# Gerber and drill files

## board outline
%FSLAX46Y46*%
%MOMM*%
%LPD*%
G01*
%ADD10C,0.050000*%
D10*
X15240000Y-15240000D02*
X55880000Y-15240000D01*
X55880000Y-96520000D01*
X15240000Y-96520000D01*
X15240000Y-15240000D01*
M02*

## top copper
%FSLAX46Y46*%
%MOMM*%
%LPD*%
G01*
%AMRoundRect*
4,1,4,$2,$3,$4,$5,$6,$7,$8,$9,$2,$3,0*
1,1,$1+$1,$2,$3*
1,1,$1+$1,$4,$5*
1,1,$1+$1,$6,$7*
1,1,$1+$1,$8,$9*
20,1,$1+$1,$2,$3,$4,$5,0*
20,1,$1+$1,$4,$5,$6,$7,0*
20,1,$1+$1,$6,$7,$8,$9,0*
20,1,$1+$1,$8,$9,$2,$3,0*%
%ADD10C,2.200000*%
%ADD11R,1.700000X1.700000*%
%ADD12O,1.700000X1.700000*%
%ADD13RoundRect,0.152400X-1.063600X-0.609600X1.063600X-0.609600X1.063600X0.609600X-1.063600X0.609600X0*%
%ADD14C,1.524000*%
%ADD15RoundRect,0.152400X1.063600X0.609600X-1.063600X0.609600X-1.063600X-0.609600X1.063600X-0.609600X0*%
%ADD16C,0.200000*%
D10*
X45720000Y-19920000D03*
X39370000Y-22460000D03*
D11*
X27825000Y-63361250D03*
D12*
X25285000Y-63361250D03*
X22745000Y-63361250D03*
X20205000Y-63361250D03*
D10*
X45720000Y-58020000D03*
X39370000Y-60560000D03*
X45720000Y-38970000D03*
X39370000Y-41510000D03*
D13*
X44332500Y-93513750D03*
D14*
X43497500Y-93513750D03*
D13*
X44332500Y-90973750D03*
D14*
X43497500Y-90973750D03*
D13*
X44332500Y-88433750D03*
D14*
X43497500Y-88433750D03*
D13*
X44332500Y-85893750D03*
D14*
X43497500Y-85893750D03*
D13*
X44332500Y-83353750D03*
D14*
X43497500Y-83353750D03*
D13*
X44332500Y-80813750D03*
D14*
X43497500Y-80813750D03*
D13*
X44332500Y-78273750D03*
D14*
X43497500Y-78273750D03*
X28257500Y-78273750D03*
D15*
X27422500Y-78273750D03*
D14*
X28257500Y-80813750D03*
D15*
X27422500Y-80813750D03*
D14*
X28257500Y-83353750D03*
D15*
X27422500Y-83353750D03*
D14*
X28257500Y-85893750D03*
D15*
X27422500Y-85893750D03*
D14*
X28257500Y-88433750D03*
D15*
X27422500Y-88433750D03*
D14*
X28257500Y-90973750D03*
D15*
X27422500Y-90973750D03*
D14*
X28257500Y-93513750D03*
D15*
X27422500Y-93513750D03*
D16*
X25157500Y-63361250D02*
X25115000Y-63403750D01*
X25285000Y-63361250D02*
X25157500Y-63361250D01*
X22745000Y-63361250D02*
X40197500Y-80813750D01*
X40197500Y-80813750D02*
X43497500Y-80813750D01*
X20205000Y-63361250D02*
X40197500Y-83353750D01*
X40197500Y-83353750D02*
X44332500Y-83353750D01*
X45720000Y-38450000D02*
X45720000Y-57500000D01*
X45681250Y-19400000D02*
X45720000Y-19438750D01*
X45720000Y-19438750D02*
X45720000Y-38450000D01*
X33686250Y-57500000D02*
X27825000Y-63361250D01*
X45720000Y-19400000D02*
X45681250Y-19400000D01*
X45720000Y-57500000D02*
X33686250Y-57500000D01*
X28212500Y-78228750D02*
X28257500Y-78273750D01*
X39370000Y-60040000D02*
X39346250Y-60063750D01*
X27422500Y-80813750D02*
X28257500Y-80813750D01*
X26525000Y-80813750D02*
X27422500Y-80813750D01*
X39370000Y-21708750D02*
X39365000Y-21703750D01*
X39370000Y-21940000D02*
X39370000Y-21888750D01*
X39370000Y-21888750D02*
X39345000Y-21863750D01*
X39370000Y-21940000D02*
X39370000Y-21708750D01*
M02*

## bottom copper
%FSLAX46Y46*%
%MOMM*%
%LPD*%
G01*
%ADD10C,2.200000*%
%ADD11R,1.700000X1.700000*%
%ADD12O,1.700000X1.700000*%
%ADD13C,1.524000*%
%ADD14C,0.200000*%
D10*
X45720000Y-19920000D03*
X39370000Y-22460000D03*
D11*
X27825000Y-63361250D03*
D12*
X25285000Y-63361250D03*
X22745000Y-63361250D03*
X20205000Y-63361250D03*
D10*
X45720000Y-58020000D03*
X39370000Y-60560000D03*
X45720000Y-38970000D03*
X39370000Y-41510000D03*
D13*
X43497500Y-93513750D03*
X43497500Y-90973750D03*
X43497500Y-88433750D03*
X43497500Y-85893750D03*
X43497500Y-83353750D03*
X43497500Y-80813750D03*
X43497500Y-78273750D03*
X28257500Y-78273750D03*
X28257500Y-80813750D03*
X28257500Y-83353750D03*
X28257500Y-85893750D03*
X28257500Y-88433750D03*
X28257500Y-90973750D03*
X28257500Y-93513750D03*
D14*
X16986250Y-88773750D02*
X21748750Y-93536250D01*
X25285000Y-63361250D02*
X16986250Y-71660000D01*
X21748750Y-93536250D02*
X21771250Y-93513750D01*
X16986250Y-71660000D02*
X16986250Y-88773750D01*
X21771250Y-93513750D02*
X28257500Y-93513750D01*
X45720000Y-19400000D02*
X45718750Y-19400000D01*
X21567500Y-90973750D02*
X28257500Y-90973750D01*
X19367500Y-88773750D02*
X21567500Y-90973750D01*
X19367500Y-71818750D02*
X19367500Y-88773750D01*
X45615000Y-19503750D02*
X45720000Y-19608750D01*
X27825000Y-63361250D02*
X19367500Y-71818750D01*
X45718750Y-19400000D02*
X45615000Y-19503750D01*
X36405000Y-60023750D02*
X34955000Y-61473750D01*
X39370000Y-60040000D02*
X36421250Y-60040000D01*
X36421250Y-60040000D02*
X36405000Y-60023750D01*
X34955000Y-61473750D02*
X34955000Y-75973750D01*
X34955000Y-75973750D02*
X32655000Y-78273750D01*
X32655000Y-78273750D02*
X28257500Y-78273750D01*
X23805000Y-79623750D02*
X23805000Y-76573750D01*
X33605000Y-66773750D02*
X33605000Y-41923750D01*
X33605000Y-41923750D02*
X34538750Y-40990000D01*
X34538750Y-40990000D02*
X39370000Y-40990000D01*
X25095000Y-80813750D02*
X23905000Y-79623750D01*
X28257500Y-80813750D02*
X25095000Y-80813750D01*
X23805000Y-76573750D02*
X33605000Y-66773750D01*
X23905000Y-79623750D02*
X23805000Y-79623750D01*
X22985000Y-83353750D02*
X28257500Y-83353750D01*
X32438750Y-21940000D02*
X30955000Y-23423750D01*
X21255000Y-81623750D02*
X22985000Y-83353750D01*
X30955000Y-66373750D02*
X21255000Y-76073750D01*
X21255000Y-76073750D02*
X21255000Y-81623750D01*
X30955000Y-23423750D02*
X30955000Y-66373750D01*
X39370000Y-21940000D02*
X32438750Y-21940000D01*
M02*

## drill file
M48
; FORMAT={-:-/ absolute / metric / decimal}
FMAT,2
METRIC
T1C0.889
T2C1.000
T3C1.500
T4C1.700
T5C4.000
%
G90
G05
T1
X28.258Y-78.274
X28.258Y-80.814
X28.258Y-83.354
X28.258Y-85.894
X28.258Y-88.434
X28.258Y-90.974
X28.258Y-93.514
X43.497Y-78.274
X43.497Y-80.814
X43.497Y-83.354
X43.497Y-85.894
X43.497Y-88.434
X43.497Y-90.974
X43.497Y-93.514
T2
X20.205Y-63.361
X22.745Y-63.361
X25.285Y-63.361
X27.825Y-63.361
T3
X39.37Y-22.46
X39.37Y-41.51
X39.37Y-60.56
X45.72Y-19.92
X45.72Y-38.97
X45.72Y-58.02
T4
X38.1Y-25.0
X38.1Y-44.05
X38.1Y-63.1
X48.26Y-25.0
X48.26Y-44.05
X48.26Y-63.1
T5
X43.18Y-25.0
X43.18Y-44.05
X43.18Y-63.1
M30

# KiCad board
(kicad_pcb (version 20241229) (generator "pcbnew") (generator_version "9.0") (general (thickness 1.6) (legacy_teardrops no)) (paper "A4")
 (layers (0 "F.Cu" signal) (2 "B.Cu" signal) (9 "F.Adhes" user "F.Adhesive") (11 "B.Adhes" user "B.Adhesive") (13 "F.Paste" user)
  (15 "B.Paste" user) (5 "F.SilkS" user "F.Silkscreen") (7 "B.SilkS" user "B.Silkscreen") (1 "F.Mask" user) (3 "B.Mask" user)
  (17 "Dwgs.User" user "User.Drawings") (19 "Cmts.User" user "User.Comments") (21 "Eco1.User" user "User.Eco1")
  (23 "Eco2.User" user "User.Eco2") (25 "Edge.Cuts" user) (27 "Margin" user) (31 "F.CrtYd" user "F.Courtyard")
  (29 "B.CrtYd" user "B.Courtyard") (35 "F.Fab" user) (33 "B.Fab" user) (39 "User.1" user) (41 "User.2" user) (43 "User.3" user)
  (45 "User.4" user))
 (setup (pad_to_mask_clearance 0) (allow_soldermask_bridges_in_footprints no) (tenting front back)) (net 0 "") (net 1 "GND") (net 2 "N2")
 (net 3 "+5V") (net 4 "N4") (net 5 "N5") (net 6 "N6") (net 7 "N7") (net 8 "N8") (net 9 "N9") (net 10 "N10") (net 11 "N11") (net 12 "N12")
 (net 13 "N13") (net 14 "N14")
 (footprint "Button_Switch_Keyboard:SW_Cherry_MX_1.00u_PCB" (layer "F.Cu") (at 45.72 19.92)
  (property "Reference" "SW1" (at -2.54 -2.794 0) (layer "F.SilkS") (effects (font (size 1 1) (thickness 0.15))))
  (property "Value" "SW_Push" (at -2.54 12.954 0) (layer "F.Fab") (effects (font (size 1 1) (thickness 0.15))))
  (pad "" np_thru_hole circle (at -7.62 5.08) (size 1.7 1.7) (drill 1.7) (layers "*.Cu" "*.Mask"))
  (pad "" np_thru_hole circle (at -2.54 5.08) (size 4 4) (drill 4) (layers "*.Cu" "*.Mask"))
  (pad "" np_thru_hole circle (at 2.54 5.08) (size 1.7 1.7) (drill 1.7) (layers "*.Cu" "*.Mask"))
  (pad "1" thru_hole circle (at 0 0) (size 2.2 2.2) (drill 1.5) (layers "*.Cu" "*.Mask") (remove_unused_layers no) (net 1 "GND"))
  (pad "2" thru_hole circle (at -6.35 2.54) (size 2.2 2.2) (drill 1.5) (layers "*.Cu" "*.Mask") (remove_unused_layers no) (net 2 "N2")))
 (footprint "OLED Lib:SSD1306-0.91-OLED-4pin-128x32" (layer "F.Cu") (at 30.015 26.86125 -90)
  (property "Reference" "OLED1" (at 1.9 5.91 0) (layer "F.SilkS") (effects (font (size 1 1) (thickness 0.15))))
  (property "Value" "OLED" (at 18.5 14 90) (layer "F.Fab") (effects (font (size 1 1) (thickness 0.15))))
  (pad "1" thru_hole rect (at 36.5 2.19 270) (size 1.7 1.7) (drill 1) (layers "*.Cu" "*.Mask") (remove_unused_layers no) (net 1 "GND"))
  (pad "2" thru_hole oval (at 36.5 4.73 270) (size 1.7 1.7) (drill 1) (layers "*.Cu" "*.Mask") (remove_unused_layers no) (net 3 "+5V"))
  (pad "3" thru_hole oval (at 36.5 7.27 270) (size 1.7 1.7) (drill 1) (layers "*.Cu" "*.Mask") (remove_unused_layers no) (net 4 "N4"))
  (pad "4" thru_hole oval (at 36.5 9.81 270) (size 1.7 1.7) (drill 1) (layers "*.Cu" "*.Mask") (remove_unused_layers no) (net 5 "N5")))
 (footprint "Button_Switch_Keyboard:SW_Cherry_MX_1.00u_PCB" (layer "F.Cu") (at 45.72 58.02)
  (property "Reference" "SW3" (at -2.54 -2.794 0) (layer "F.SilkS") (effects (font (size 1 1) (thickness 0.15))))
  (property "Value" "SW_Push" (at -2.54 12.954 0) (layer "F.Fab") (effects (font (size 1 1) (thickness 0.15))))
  (pad "" np_thru_hole circle (at -7.62 5.08) (size 1.7 1.7) (drill 1.7) (layers "*.Cu" "*.Mask"))
  (pad "" np_thru_hole circle (at -2.54 5.08) (size 4 4) (drill 4) (layers "*.Cu" "*.Mask"))
  (pad "" np_thru_hole circle (at 2.54 5.08) (size 1.7 1.7) (drill 1.7) (layers "*.Cu" "*.Mask"))
  (pad "1" thru_hole circle (at 0 0) (size 2.2 2.2) (drill 1.5) (layers "*.Cu" "*.Mask") (remove_unused_layers no) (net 1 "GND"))
  (pad "2" thru_hole circle (at -6.35 2.54) (size 2.2 2.2) (drill 1.5) (layers "*.Cu" "*.Mask") (remove_unused_layers no) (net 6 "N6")))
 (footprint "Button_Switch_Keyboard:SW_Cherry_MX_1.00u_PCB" (layer "F.Cu") (at 45.72 38.97)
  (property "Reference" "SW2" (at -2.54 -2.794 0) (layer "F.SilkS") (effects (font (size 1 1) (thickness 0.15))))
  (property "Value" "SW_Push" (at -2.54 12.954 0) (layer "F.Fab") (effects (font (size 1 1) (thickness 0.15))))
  (pad "" np_thru_hole circle (at -7.62 5.08) (size 1.7 1.7) (drill 1.7) (layers "*.Cu" "*.Mask"))
  (pad "" np_thru_hole circle (at -2.54 5.08) (size 4 4) (drill 4) (layers "*.Cu" "*.Mask"))
  (pad "" np_thru_hole circle (at 2.54 5.08) (size 1.7 1.7) (drill 1.7) (layers "*.Cu" "*.Mask"))
  (pad "1" thru_hole circle (at 0 0) (size 2.2 2.2) (drill 1.5) (layers "*.Cu" "*.Mask") (remove_unused_layers no) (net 1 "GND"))
  (pad "2" thru_hole circle (at -6.35 2.54) (size 2.2 2.2) (drill 1.5) (layers "*.Cu" "*.Mask") (remove_unused_layers no) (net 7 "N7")))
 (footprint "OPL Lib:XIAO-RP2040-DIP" (layer "F.Cu") (at 35.8775 85.89375 180)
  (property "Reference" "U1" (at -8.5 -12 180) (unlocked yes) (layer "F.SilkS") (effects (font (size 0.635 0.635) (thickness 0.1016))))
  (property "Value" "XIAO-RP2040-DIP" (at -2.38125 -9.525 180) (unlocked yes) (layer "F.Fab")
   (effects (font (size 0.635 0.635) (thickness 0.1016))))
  (pad "1" smd roundrect (at -8.455 -7.62) (size 2.432 1.524) (layers "F.Cu" "F.Mask") (roundrect_rratio 0.1) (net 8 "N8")
   (thermal_bridge_angle 45))
  (pad "1" thru_hole circle (at -7.62 -7.62) (size 1.524 1.524) (drill 0.889) (layers "*.Cu" "*.Mask") (remove_unused_layers no)
   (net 8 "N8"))
  (pad "2" smd roundrect (at -8.455 -5.08) (size 2.432 1.524) (layers "F.Cu" "F.Mask") (roundrect_rratio 0.1) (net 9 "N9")
   (thermal_bridge_angle 45))
  (pad "2" thru_hole circle (at -7.62 -5.08) (size 1.524 1.524) (drill 0.889) (layers "*.Cu" "*.Mask") (remove_unused_layers no)
   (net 9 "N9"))
  (pad "3" smd roundrect (at -8.455 -2.54) (size 2.432 1.524) (layers "F.Cu" "F.Mask") (roundrect_rratio 0.1) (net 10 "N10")
   (thermal_bridge_angle 45))
  (pad "3" thru_hole circle (at -7.62 -2.54) (size 1.524 1.524) (drill 0.889) (layers "*.Cu" "*.Mask") (remove_unused_layers no)
   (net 10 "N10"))
  (pad "4" smd roundrect (at -8.455 0) (size 2.432 1.524) (layers "F.Cu" "F.Mask") (roundrect_rratio 0.1) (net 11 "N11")
   (thermal_bridge_angle 45))
  (pad "4" thru_hole circle (at -7.62 0) (size 1.524 1.524) (drill 0.889) (layers "*.Cu" "*.Mask") (remove_unused_layers no) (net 11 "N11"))
  (pad "5" smd roundrect (at -8.455 2.54) (size 2.432 1.524) (layers "F.Cu" "F.Mask") (roundrect_rratio 0.1) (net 5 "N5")
   (thermal_bridge_angle 45))
  (pad "5" thru_hole circle (at -7.62 2.54) (size 1.524 1.524) (drill 0.889) (layers "*.Cu" "*.Mask") (remove_unused_layers no) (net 5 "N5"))
  (pad "6" smd roundrect (at -8.455 5.08) (size 2.432 1.524) (layers "F.Cu" "F.Mask") (roundrect_rratio 0.1) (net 4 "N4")
   (thermal_bridge_angle 45))
  (pad "6" thru_hole circle (at -7.62 5.08) (size 1.524 1.524) (drill 0.889) (layers "*.Cu" "*.Mask") (remove_unused_layers no) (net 4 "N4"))
  (pad "7" smd roundrect (at -8.455 7.62) (size 2.432 1.524) (layers "F.Cu" "F.Mask") (roundrect_rratio 0.1) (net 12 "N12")
   (thermal_bridge_angle 45))
  (pad "7" thru_hole circle (at -7.62 7.62) (size 1.524 1.524) (drill 0.889) (layers "*.Cu" "*.Mask") (remove_unused_layers no)
   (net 12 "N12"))
  (pad "8" thru_hole circle (at 7.62 7.62 180) (size 1.524 1.524) (drill 0.889) (layers "*.Cu" "*.Mask") (remove_unused_layers no)
   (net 6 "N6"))
  (pad "8" smd roundrect (at 8.455 7.62 180) (size 2.432 1.524) (layers "F.Cu" "F.Mask") (roundrect_rratio 0.1) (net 6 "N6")
   (thermal_bridge_angle 45))
  (pad "9" thru_hole circle (at 7.62 5.08 180) (size 1.524 1.524) (drill 0.889) (layers "*.Cu" "*.Mask") (remove_unused_layers no)
   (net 7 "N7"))
  (pad "9" smd roundrect (at 8.455 5.08 180) (size 2.432 1.524) (layers "F.Cu" "F.Mask") (roundrect_rratio 0.1) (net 7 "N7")
   (thermal_bridge_angle 45))
  (pad "10" thru_hole circle (at 7.62 2.54 180) (size 1.524 1.524) (drill 0.889) (layers "*.Cu" "*.Mask") (remove_unused_layers no)
   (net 2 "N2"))
  (pad "10" smd roundrect (at 8.455 2.54 180) (size 2.432 1.524) (layers "F.Cu" "F.Mask") (roundrect_rratio 0.1) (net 2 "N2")
   (thermal_bridge_angle 45))
  (pad "11" thru_hole circle (at 7.62 0 180) (size 1.524 1.524) (drill 0.889) (layers "*.Cu" "*.Mask") (remove_unused_layers no)
   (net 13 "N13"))
  (pad "11" smd roundrect (at 8.455 0 180) (size 2.432 1.524) (layers "F.Cu" "F.Mask") (roundrect_rratio 0.1) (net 13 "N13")
   (thermal_bridge_angle 45))
  (pad "12" thru_hole circle (at 7.62 -2.54 180) (size 1.524 1.524) (drill 0.889) (layers "*.Cu" "*.Mask") (remove_unused_layers no)
   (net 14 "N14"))
  (pad "12" smd roundrect (at 8.455 -2.54 180) (size 2.432 1.524) (layers "F.Cu" "F.Mask") (roundrect_rratio 0.1) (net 14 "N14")
   (thermal_bridge_angle 45))
  (pad "13" thru_hole circle (at 7.62 -5.08 180) (size 1.524 1.524) (drill 0.889) (layers "*.Cu" "*.Mask") (remove_unused_layers no)
   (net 1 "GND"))
  (pad "13" smd roundrect (at 8.455 -5.08 180) (size 2.432 1.524) (layers "F.Cu" "F.Mask") (roundrect_rratio 0.1) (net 1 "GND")
   (thermal_bridge_angle 45))
  (pad "14" thru_hole circle (at 7.62 -7.62 180) (size 1.524 1.524) (drill 0.889) (layers "*.Cu" "*.Mask") (remove_unused_layers no)
   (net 3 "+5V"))
  (pad "14" smd roundrect (at 8.455 -7.62 180) (size 2.432 1.524) (layers "F.Cu" "F.Mask") (roundrect_rratio 0.1) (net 3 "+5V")
   (thermal_bridge_angle 45)))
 (gr_rect (start 15.24 15.24) (end 55.88 96.52) (stroke (width 0.05) (type solid)) (fill no) (layer "Edge.Cuts"))
 (segment (start 25.1575 63.36125) (end 25.115 63.40375) (width 0.2) (layer "F.Cu") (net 3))
 (segment (start 25.285 63.36125) (end 25.1575 63.36125) (width 0.2) (layer "F.Cu") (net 3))
 (segment (start 16.98625 88.77375) (end 21.74875 93.53625) (width 0.2) (layer "B.Cu") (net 3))
 (segment (start 25.285 63.36125) (end 16.98625 71.66) (width 0.2) (layer "B.Cu") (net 3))
 (segment (start 21.74875 93.53625) (end 21.77125 93.51375) (width 0.2) (layer "B.Cu") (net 3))
 (segment (start 16.98625 71.66) (end 16.98625 88.77375) (width 0.2) (layer "B.Cu") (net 3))
 (segment (start 21.77125 93.51375) (end 28.2575 93.51375) (width 0.2) (layer "B.Cu") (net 3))
 (segment (start 22.745 63.36125) (end 40.1975 80.81375) (width 0.2) (layer "F.Cu") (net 4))
 (segment (start 40.1975 80.81375) (end 43.4975 80.81375) (width 0.2) (layer "F.Cu") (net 4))
 (segment (start 20.205 63.36125) (end 40.1975 83.35375) (width 0.2) (layer "F.Cu") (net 5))
 (segment (start 40.1975 83.35375) (end 44.3325 83.35375) (width 0.2) (layer "F.Cu") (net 5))
 (segment (start 45.72 38.45) (end 45.72 57.5) (width 0.2) (layer "F.Cu") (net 1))
 (segment (start 45.68125 19.4) (end 45.72 19.43875) (width 0.2) (layer "F.Cu") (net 1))
 (segment (start 45.72 19.43875) (end 45.72 38.45) (width 0.2) (layer "F.Cu") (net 1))
 (segment (start 33.68625 57.5) (end 27.825 63.36125) (width 0.2) (layer "F.Cu") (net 1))
 (segment (start 45.72 19.4) (end 45.68125 19.4) (width 0.2) (layer "F.Cu") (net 1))
 (segment (start 45.72 57.5) (end 33.68625 57.5) (width 0.2) (layer "F.Cu") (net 1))
 (segment (start 45.72 19.4) (end 45.71875 19.4) (width 0.2) (layer "B.Cu") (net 1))
 (segment (start 21.5675 90.97375) (end 28.2575 90.97375) (width 0.2) (layer "B.Cu") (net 1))
 (segment (start 19.3675 88.77375) (end 21.5675 90.97375) (width 0.2) (layer "B.Cu") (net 1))
 (segment (start 19.3675 71.81875) (end 19.3675 88.77375) (width 0.2) (layer "B.Cu") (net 1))
 (segment (start 45.615 19.50375) (end 45.72 19.60875) (width 0.2) (layer "B.Cu") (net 1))
 (segment (start 27.825 63.36125) (end 19.3675 71.81875) (width 0.2) (layer "B.Cu") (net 1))
 (segment (start 45.71875 19.4) (end 45.615 19.50375) (width 0.2) (layer "B.Cu") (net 1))
 (segment (start 28.2125 78.22875) (end 28.2575 78.27375) (width 0.2) (layer "F.Cu") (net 6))
 (segment (start 39.37 60.04) (end 39.34625 60.06375) (width 0.2) (layer "F.Cu") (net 6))
 (segment (start 36.405 60.02375) (end 34.955 61.47375) (width 0.2) (layer "B.Cu") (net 6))
 (segment (start 39.37 60.04) (end 36.42125 60.04) (width 0.2) (layer "B.Cu") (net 6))
 (segment (start 36.42125 60.04) (end 36.405 60.02375) (width 0.2) (layer "B.Cu") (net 6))
 (segment (start 34.955 61.47375) (end 34.955 75.97375) (width 0.2) (layer "B.Cu") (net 6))
 (segment (start 34.955 75.97375) (end 32.655 78.27375) (width 0.2) (layer "B.Cu") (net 6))
 (segment (start 32.655 78.27375) (end 28.2575 78.27375) (width 0.2) (layer "B.Cu") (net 6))
 (segment (start 27.4225 80.81375) (end 28.2575 80.81375) (width 0.2) (layer "F.Cu") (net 7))
 (segment (start 26.525 80.81375) (end 27.4225 80.81375) (width 0.2) (layer "F.Cu") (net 7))
 (segment (start 23.805 79.62375) (end 23.805 76.57375) (width 0.2) (layer "B.Cu") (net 7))
 (segment (start 33.605 66.77375) (end 33.605 41.92375) (width 0.2) (layer "B.Cu") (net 7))
 (segment (start 33.605 41.92375) (end 34.53875 40.99) (width 0.2) (layer "B.Cu") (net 7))
 (segment (start 34.53875 40.99) (end 39.37 40.99) (width 0.2) (layer "B.Cu") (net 7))
 (segment (start 25.095 80.81375) (end 23.905 79.62375) (width 0.2) (layer "B.Cu") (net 7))
 (segment (start 28.2575 80.81375) (end 25.095 80.81375) (width 0.2) (layer "B.Cu") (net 7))
 (segment (start 23.805 76.57375) (end 33.605 66.77375) (width 0.2) (layer "B.Cu") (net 7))
 (segment (start 23.905 79.62375) (end 23.805 79.62375) (width 0.2) (layer "B.Cu") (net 7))
 (segment (start 39.37 21.70875) (end 39.365 21.70375) (width 0.2) (layer "F.Cu") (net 2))
 (segment (start 39.37 21.94) (end 39.37 21.88875) (width 0.2) (layer "F.Cu") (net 2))
 (segment (start 39.37 21.88875) (end 39.345 21.86375) (width 0.2) (layer "F.Cu") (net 2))
 (segment (start 39.37 21.94) (end 39.37 21.70875) (width 0.2) (layer "F.Cu") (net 2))
 (segment (start 22.985 83.35375) (end 28.2575 83.35375) (width 0.2) (layer "B.Cu") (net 2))
 (segment (start 32.43875 21.94) (end 30.955 23.42375) (width 0.2) (layer "B.Cu") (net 2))
 (segment (start 21.255 81.62375) (end 22.985 83.35375) (width 0.2) (layer "B.Cu") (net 2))
 (segment (start 30.955 66.37375) (end 21.255 76.07375) (width 0.2) (layer "B.Cu") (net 2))
 (segment (start 21.255 76.07375) (end 21.255 81.62375) (width 0.2) (layer "B.Cu") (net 2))
 (segment (start 30.955 23.42375) (end 30.955 66.37375) (width 0.2) (layer "B.Cu") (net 2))
 (segment (start 39.37 21.94) (end 32.43875 21.94) (width 0.2) (layer "B.Cu") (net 2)))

